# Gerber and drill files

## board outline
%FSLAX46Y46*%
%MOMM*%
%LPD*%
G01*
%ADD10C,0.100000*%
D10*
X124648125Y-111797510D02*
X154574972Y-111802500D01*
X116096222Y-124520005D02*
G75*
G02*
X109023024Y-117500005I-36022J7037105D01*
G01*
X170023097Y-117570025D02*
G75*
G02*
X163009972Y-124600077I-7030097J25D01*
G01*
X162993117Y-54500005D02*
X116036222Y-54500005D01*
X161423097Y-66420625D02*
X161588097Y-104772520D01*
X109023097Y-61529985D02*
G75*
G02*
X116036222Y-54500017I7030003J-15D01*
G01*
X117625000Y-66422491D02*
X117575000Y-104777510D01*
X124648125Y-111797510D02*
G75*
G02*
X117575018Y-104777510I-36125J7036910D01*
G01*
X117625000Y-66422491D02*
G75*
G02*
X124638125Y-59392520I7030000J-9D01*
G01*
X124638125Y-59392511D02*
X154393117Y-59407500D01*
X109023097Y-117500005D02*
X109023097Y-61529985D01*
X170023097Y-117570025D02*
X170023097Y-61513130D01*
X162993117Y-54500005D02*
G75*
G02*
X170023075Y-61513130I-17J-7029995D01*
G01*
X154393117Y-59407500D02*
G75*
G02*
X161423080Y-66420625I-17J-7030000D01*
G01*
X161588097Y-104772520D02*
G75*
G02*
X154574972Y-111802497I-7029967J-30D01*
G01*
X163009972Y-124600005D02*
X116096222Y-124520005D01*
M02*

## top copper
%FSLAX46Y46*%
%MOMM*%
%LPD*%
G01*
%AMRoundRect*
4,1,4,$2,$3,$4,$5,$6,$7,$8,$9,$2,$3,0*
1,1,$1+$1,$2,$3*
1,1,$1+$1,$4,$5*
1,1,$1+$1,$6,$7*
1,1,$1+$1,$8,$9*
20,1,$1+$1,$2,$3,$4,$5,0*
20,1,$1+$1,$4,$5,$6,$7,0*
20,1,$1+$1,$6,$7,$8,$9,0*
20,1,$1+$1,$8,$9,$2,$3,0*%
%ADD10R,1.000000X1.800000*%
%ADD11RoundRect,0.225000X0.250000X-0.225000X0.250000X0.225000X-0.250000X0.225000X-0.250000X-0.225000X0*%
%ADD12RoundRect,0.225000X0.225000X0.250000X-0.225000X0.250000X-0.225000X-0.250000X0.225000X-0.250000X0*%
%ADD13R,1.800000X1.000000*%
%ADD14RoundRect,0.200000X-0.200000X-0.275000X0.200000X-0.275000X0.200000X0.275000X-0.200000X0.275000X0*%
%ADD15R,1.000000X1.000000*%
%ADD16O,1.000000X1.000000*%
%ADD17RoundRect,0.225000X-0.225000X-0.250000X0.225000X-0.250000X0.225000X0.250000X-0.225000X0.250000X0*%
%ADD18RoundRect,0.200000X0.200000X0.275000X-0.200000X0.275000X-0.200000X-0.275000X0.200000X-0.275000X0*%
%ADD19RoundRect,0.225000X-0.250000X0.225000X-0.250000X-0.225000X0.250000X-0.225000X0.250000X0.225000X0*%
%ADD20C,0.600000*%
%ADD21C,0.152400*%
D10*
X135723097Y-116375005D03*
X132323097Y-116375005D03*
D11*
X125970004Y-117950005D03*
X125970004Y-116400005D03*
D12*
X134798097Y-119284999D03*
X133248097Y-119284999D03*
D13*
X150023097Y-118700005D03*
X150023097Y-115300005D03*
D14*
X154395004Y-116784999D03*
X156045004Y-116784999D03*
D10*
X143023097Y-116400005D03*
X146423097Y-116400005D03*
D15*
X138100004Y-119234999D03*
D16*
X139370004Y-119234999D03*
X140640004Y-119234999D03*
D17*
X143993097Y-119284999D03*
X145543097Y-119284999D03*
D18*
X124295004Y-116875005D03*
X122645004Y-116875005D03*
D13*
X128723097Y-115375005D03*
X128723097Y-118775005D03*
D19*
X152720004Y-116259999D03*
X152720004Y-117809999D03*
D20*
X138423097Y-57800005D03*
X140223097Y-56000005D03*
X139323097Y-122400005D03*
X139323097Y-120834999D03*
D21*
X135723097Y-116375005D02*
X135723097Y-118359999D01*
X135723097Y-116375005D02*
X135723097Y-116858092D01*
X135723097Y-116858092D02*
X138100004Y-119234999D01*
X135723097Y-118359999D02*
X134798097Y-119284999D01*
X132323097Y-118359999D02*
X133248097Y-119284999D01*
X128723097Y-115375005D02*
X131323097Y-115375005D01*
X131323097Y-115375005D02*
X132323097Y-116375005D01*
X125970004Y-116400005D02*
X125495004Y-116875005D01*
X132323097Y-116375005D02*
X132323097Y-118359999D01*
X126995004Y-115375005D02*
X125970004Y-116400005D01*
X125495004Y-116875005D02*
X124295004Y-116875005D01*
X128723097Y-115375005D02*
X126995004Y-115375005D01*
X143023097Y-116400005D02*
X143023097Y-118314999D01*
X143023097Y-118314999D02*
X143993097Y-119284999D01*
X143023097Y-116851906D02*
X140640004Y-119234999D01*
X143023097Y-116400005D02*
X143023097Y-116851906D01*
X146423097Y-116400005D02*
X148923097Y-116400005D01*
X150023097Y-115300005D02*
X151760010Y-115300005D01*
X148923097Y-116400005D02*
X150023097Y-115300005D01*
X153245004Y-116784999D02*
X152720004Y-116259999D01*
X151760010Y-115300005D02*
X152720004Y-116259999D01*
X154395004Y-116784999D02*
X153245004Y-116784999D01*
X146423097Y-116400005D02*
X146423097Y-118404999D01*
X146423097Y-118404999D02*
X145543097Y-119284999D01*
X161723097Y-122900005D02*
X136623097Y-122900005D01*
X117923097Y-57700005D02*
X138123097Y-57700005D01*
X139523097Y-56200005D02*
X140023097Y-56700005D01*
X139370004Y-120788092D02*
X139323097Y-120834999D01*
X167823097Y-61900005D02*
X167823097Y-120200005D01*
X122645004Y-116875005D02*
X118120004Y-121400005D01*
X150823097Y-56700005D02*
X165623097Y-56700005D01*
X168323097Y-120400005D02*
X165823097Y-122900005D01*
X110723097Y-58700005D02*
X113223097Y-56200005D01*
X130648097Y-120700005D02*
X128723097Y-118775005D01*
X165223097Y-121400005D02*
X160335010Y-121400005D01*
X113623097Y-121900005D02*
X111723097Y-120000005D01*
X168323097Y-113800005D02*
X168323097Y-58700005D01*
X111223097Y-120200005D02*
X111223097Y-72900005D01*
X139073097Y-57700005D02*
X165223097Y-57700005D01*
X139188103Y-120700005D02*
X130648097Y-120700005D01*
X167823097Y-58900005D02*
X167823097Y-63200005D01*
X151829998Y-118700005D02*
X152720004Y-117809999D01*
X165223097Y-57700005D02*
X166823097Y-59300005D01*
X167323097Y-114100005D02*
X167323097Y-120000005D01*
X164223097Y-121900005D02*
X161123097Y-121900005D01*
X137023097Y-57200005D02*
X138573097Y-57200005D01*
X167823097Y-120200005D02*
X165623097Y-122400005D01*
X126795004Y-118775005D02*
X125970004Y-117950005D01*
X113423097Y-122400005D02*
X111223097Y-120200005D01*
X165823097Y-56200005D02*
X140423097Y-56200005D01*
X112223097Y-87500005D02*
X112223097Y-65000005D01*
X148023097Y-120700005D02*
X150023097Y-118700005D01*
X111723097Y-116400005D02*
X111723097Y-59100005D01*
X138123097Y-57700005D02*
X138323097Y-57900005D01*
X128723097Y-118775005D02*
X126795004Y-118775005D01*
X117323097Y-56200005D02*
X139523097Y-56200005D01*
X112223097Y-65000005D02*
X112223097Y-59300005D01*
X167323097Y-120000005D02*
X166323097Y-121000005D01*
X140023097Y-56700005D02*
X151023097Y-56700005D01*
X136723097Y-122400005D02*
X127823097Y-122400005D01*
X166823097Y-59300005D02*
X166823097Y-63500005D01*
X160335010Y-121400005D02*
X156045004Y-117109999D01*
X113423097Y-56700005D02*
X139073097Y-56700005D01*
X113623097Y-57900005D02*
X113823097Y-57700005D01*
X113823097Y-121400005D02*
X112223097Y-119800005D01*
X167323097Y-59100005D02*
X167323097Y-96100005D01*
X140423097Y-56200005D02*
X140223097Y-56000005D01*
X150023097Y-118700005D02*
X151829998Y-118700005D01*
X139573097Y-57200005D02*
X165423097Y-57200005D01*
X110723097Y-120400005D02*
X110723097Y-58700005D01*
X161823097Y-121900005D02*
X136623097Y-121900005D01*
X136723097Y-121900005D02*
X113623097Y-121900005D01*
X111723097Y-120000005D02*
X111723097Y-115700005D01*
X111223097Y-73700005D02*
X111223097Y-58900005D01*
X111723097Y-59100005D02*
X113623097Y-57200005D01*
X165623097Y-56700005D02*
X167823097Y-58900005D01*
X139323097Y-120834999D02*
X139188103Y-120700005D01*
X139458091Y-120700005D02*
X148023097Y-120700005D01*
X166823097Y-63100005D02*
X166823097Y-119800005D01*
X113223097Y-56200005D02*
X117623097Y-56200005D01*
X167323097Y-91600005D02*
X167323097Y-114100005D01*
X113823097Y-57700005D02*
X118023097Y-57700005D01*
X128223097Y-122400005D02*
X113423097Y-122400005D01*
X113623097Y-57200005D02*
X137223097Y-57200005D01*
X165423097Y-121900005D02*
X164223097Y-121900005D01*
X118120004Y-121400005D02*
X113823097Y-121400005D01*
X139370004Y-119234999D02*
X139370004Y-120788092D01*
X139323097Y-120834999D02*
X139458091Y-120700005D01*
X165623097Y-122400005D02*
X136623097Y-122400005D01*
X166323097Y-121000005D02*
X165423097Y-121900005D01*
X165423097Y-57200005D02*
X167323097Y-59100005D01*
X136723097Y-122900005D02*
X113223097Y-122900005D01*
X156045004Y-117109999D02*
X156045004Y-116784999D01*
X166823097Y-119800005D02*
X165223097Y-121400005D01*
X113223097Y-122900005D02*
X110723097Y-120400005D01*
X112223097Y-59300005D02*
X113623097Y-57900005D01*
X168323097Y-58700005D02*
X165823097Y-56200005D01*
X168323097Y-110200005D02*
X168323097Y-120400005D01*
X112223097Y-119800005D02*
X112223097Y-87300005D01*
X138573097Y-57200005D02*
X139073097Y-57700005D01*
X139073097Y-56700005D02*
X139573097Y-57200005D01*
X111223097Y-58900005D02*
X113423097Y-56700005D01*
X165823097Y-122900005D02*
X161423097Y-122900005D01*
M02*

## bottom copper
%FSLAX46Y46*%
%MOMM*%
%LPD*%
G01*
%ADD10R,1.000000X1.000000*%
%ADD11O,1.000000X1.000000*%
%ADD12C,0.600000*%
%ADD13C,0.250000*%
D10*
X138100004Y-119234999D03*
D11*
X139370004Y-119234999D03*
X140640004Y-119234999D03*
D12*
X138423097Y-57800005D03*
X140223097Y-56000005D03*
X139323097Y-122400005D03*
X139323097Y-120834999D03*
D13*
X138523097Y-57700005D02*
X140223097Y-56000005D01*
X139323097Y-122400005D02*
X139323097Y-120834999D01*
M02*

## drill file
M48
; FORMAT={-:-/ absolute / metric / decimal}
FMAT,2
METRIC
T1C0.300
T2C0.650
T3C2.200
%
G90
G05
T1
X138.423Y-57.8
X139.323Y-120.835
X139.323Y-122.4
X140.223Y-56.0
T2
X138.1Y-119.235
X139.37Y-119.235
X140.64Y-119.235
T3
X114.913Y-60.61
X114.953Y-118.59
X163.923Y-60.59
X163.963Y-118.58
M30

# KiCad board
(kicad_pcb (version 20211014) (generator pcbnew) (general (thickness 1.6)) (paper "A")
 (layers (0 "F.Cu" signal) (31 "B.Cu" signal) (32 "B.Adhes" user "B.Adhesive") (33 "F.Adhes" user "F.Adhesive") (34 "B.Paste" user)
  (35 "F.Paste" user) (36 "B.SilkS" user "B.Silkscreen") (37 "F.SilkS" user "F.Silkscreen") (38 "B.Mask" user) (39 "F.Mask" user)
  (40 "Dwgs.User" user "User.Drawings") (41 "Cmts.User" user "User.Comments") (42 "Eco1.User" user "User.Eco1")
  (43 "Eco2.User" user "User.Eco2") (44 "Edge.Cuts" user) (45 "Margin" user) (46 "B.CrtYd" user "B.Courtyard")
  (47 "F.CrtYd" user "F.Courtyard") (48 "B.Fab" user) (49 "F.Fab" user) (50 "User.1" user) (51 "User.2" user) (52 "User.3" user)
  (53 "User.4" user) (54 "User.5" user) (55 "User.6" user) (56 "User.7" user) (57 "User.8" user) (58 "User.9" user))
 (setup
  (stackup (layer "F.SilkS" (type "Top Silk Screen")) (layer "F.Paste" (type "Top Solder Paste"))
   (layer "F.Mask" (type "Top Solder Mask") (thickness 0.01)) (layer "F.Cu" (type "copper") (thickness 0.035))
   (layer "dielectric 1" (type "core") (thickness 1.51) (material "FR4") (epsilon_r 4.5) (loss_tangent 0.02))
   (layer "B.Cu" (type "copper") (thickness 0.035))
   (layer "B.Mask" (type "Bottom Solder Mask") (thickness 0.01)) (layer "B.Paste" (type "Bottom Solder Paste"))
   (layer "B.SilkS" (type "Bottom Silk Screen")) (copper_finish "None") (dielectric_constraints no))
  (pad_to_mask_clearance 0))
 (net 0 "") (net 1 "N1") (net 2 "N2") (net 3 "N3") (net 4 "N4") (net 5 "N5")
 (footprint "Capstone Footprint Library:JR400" (layer "F.Cu") (at 134.023097 116.375005 180)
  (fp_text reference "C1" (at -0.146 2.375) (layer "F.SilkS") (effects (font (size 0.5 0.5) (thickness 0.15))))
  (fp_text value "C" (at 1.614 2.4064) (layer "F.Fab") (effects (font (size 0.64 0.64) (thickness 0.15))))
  (pad "1" smd rect (at -1.7 0 180) (size 1 1.8) (layers "F.Cu" "F.Paste" "F.Mask") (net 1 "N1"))
  (pad "2" smd rect (at 1.7 0 180) (size 1 1.8) (layers "F.Cu" "F.Paste" "F.Mask") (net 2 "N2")))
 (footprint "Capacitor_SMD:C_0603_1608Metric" (layer "F.Cu") (at 125.970004 117.175005 90)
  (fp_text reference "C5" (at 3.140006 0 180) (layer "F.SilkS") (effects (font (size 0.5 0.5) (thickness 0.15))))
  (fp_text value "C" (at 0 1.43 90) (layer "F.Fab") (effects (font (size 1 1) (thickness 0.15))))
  (pad "1" smd roundrect (at -0.775 0 90) (size 0.9 0.95) (layers "F.Cu" "F.Paste" "F.Mask") (roundrect_rratio 0.25) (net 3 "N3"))
  (pad "2" smd roundrect (at 0.775 0 90) (size 0.9 0.95) (layers "F.Cu" "F.Paste" "F.Mask") (roundrect_rratio 0.25) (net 2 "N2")))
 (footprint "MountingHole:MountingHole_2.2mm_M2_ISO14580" (layer "F.Cu") (at 163.923097 60.590005)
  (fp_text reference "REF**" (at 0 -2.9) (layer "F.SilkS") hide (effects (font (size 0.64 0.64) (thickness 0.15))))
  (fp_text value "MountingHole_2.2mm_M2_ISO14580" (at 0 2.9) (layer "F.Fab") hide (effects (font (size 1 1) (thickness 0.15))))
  (pad "" np_thru_hole circle (at 0 0) (size 2.2 2.2) (drill 2.2) (layers *.Cu *.Mask)))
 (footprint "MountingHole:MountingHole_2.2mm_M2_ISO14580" (layer "F.Cu") (at 163.963097 118.580005)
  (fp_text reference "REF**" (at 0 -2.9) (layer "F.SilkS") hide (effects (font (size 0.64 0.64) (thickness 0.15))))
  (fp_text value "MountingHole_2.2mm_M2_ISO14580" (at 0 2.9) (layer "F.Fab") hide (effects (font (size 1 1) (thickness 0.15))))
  (pad "" np_thru_hole circle (at 0 0) (size 2.2 2.2) (drill 2.2) (layers *.Cu *.Mask)))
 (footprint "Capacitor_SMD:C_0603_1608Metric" (layer "F.Cu") (at 134.023097 119.284999 180)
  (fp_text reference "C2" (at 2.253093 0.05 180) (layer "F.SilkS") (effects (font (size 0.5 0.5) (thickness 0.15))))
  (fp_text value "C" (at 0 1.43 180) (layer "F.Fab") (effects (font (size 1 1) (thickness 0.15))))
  (pad "1" smd roundrect (at -0.775 0 180) (size 0.9 0.95) (layers "F.Cu" "F.Paste" "F.Mask") (roundrect_rratio 0.25) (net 1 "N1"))
  (pad "2" smd roundrect (at 0.775 0 180) (size 0.9 0.95) (layers "F.Cu" "F.Paste" "F.Mask") (roundrect_rratio 0.25) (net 2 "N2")))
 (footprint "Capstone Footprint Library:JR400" (layer "F.Cu") (at 150.023097 117.000005 90)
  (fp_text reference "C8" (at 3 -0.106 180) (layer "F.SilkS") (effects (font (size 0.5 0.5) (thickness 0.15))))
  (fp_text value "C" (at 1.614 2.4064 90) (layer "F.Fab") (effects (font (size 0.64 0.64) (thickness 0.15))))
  (pad "1" smd rect (at -1.7 0 90) (size 1 1.8) (layers "F.Cu" "F.Paste" "F.Mask") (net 3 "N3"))
  (pad "2" smd rect (at 1.7 0 90) (size 1 1.8) (layers "F.Cu" "F.Paste" "F.Mask") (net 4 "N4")))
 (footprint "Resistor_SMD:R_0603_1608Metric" (layer "F.Cu") (at 155.220004 116.784999)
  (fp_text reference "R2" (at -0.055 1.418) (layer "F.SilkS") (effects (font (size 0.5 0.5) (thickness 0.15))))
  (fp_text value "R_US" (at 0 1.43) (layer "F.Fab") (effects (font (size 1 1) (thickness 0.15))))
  (pad "1" smd roundrect (at -0.825 0) (size 0.8 0.95) (layers "F.Cu" "F.Paste" "F.Mask") (roundrect_rratio 0.25) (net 4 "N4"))
  (pad "2" smd roundrect (at 0.825 0) (size 0.8 0.95) (layers "F.Cu" "F.Paste" "F.Mask") (roundrect_rratio 0.25) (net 3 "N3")))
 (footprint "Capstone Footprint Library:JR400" (layer "F.Cu") (at 144.723097 116.400005)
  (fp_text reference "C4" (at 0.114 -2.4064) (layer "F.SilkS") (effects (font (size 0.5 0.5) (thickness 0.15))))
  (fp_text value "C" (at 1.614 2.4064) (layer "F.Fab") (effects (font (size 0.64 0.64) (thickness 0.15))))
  (pad "1" smd rect (at -1.7 0) (size 1 1.8) (layers "F.Cu" "F.Paste" "F.Mask") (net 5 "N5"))
  (pad "2" smd rect (at 1.7 0) (size 1 1.8) (layers "F.Cu" "F.Paste" "F.Mask") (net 4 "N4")))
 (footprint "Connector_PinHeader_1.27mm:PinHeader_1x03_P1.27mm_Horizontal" (layer "F.Cu") (at 138.100004 119.234999 90)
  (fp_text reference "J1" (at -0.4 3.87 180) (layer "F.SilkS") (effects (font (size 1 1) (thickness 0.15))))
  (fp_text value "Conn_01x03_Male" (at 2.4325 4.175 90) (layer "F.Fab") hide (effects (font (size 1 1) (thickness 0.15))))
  (pad "1" thru_hole rect (at 0 0 90) (size 1 1) (drill 0.65) (layers *.Cu *.Mask) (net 1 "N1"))
  (pad "2" thru_hole oval (at 0 1.27 90) (size 1 1) (drill 0.65) (layers *.Cu *.Mask) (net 3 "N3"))
  (pad "3" thru_hole oval (at 0 2.54 90) (size 1 1) (drill 0.65) (layers *.Cu *.Mask) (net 5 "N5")))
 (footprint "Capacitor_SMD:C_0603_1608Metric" (layer "F.Cu") (at 144.768097 119.284999)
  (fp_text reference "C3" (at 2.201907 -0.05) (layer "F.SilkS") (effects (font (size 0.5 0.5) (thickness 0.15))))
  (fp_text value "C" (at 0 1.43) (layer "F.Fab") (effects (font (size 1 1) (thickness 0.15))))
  (pad "1" smd roundrect (at -0.775 0) (size 0.9 0.95) (layers "F.Cu" "F.Paste" "F.Mask") (roundrect_rratio 0.25) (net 5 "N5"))
  (pad "2" smd roundrect (at 0.775 0) (size 0.9 0.95) (layers "F.Cu" "F.Paste" "F.Mask") (roundrect_rratio 0.25) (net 4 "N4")))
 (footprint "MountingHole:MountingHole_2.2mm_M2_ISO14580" (layer "F.Cu") (at 114.953097 118.590005)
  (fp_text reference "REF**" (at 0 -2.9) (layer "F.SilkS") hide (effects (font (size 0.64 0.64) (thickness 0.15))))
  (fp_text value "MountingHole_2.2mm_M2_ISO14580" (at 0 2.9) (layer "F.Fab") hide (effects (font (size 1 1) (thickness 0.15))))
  (pad "" np_thru_hole circle (at 0 0) (size 2.2 2.2) (drill 2.2) (layers *.Cu *.Mask)))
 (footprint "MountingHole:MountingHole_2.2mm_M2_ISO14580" (layer "F.Cu") (at 114.913097 60.610005)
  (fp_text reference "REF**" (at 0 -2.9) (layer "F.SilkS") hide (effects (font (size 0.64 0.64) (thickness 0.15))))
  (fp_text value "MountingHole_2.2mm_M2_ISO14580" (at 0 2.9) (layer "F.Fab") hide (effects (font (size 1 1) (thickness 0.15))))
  (pad "" np_thru_hole circle (at 0 0) (size 2.2 2.2) (drill 2.2) (layers *.Cu *.Mask)))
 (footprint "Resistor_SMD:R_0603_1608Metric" (layer "F.Cu") (at 123.470004 116.875005 180)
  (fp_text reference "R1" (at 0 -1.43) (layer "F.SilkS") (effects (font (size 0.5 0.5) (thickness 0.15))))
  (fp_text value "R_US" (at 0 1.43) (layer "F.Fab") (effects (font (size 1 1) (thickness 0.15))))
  (pad "1" smd roundrect (at -0.825 0 180) (size 0.8 0.95) (layers "F.Cu" "F.Paste" "F.Mask") (roundrect_rratio 0.25) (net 2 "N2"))
  (pad "2" smd roundrect (at 0.825 0 180) (size 0.8 0.95) (layers "F.Cu" "F.Paste" "F.Mask") (roundrect_rratio 0.25) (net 3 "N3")))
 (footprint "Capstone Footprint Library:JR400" (layer "F.Cu") (at 128.723097 117.075005 -90)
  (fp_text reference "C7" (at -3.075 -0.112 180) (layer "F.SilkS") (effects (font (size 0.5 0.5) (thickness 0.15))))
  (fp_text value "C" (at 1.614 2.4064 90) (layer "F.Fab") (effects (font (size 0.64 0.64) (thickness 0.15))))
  (pad "1" smd rect (at -1.7 0 270) (size 1 1.8) (layers "F.Cu" "F.Paste" "F.Mask") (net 2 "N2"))
  (pad "2" smd rect (at 1.7 0 270) (size 1 1.8) (layers "F.Cu" "F.Paste" "F.Mask") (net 3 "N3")))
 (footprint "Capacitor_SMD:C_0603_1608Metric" (layer "F.Cu") (at 152.720004 117.034999 -90)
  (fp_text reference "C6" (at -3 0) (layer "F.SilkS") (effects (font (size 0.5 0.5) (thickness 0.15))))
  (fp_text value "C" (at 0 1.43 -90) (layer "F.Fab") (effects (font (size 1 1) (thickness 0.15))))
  (pad "1" smd roundrect (at -0.775 0 270) (size 0.9 0.95) (layers "F.Cu" "F.Paste" "F.Mask") (roundrect_rratio 0.25) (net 4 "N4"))
  (pad "2" smd roundrect (at 0.775 0 270) (size 0.9 0.95) (layers "F.Cu" "F.Paste" "F.Mask") (roundrect_rratio 0.25) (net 3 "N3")))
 (gr_line (start 124.648125 111.79751) (end 154.574972 111.8025) (layer "Edge.Cuts") (width 0.1))
 (gr_arc (start 116.096222 124.520005) (mid 111.103006 122.47769) (end 109.023097 117.500005) (layer "Edge.Cuts") (width 0.1))
 (gr_arc (start 170.023097 117.570025) (mid 167.970004 122.535002) (end 163.009972 124.600005) (layer "Edge.Cuts") (width 0.1))
 (gr_line (start 162.993117 54.500005) (end 116.036222 54.500005) (layer "Edge.Cuts") (width 0.1))
 (gr_line (start 161.423097 66.420625) (end 161.588097 104.77252) (layer "Edge.Cuts") (width 0.1))
 (gr_arc (start 109.023097 61.529985) (mid 111.076178 56.565001) (end 116.036222 54.500005) (layer "Edge.Cuts") (width 0.1))
 (gr_line (start 117.625 66.422491) (end 117.575 104.77751) (layer "Edge.Cuts") (width 0.1))
 (gr_arc (start 124.648125 111.79751) (mid 119.654876 109.755226) (end 117.575 104.77751) (layer "Edge.Cuts") (width 0.1))
 (gr_arc (start 117.625 66.422491) (mid 119.678079 61.457504) (end 124.638125 59.392511) (layer "Edge.Cuts") (width 0.1))
 (gr_line (start 124.638125 59.392511) (end 154.393117 59.4075) (layer "Edge.Cuts") (width 0.1))
 (gr_line (start 109.023097 117.500005) (end 109.023097 61.529985) (layer "Edge.Cuts") (width 0.1))
 (gr_line (start 170.023097 117.570025) (end 170.023097 61.51313) (layer "Edge.Cuts") (width 0.1))
 (gr_arc (start 162.993117 54.500005) (mid 167.958097 56.553087) (end 170.023097 61.51313) (layer "Edge.Cuts") (width 0.1))
 (gr_arc (start 154.393117 59.4075) (mid 159.358099 61.460581) (end 161.423097 66.420625) (layer "Edge.Cuts") (width 0.1))
 (gr_arc (start 161.588097 104.77252) (mid 159.535019 109.73753) (end 154.574972 111.8025) (layer "Edge.Cuts") (width 0.1))
 (gr_line (start 163.009972 124.600005) (end 116.096222 124.520005) (layer "Edge.Cuts") (width 0.1))
 (segment (start 135.723097 116.375005) (end 135.723097 118.359999) (width 0.1524) (layer "F.Cu") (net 1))
 (segment (start 135.723097 116.375005) (end 135.723097 116.858092) (width 0.1524) (layer "F.Cu") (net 1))
 (segment (start 135.723097 116.858092) (end 138.100004 119.234999) (width 0.1524) (layer "F.Cu") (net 1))
 (segment (start 135.723097 118.359999) (end 134.798097 119.284999) (width 0.1524) (layer "F.Cu") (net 1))
 (segment (start 132.323097 118.359999) (end 133.248097 119.284999) (width 0.1524) (layer "F.Cu") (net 2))
 (segment (start 128.723097 115.375005) (end 131.323097 115.375005) (width 0.1524) (layer "F.Cu") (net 2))
 (segment (start 131.323097 115.375005) (end 132.323097 116.375005) (width 0.1524) (layer "F.Cu") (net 2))
 (segment (start 125.970004 116.400005) (end 125.495004 116.875005) (width 0.1524) (layer "F.Cu") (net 2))
 (segment (start 132.323097 116.375005) (end 132.323097 118.359999) (width 0.1524) (layer "F.Cu") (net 2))
 (segment (start 126.995004 115.375005) (end 125.970004 116.400005) (width 0.1524) (layer "F.Cu") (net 2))
 (segment (start 125.495004 116.875005) (end 124.295004 116.875005) (width 0.1524) (layer "F.Cu") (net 2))
 (segment (start 128.723097 115.375005) (end 126.995004 115.375005) (width 0.1524) (layer "F.Cu") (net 2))
 (segment (start 143.023097 116.400005) (end 143.023097 118.314999) (width 0.1524) (layer "F.Cu") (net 5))
 (segment (start 143.023097 118.314999) (end 143.993097 119.284999) (width 0.1524) (layer "F.Cu") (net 5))
 (segment (start 143.023097 116.851906) (end 140.640004 119.234999) (width 0.1524) (layer "F.Cu") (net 5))
 (segment (start 143.023097 116.400005) (end 143.023097 116.851906) (width 0.1524) (layer "F.Cu") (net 5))
 (segment (start 146.423097 116.400005) (end 148.923097 116.400005) (width 0.1524) (layer "F.Cu") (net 4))
 (segment (start 150.023097 115.300005) (end 151.76001 115.300005) (width 0.1524) (layer "F.Cu") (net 4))
 (segment (start 148.923097 116.400005) (end 150.023097 115.300005) (width 0.1524) (layer "F.Cu") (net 4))
 (segment (start 153.245004 116.784999) (end 152.720004 116.259999) (width 0.1524) (layer "F.Cu") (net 4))
 (segment (start 151.76001 115.300005) (end 152.720004 116.259999) (width 0.1524) (layer "F.Cu") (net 4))
 (segment (start 154.395004 116.784999) (end 153.245004 116.784999) (width 0.1524) (layer "F.Cu") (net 4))
 (segment (start 146.423097 116.400005) (end 146.423097 118.404999) (width 0.1524) (layer "F.Cu") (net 4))
 (segment (start 146.423097 118.404999) (end 145.543097 119.284999) (width 0.1524) (layer "F.Cu") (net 4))
 (segment (start 161.723097 122.900005) (end 136.623097 122.900005) (width 0.1524) (layer "F.Cu") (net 3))
 (segment (start 117.923097 57.700005) (end 138.123097 57.700005) (width 0.1524) (layer "F.Cu") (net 3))
 (segment (start 139.523097 56.200005) (end 140.023097 56.700005) (width 0.1524) (layer "F.Cu") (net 3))
 (segment (start 139.370004 120.788092) (end 139.323097 120.834999) (width 0.1524) (layer "F.Cu") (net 3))
 (segment (start 167.823097 61.900005) (end 167.823097 120.200005) (width 0.1524) (layer "F.Cu") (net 3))
 (segment (start 122.645004 116.875005) (end 118.120004 121.400005) (width 0.1524) (layer "F.Cu") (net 3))
 (segment (start 150.823097 56.700005) (end 165.623097 56.700005) (width 0.1524) (layer "F.Cu") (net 3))
 (segment (start 168.323097 120.400005) (end 165.823097 122.900005) (width 0.1524) (layer "F.Cu") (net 3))
 (segment (start 110.723097 58.700005) (end 113.223097 56.200005) (width 0.1524) (layer "F.Cu") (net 3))
 (segment (start 130.648097 120.700005) (end 128.723097 118.775005) (width 0.1524) (layer "F.Cu") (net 3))
 (segment (start 165.223097 121.400005) (end 160.33501 121.400005) (width 0.1524) (layer "F.Cu") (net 3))
 (segment (start 113.623097 121.900005) (end 111.723097 120.000005) (width 0.1524) (layer "F.Cu") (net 3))
 (segment (start 168.323097 113.800005) (end 168.323097 58.700005) (width 0.1524) (layer "F.Cu") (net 3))
 (segment (start 111.223097 120.200005) (end 111.223097 72.900005) (width 0.1524) (layer "F.Cu") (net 3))
 (segment (start 139.073097 57.700005) (end 165.223097 57.700005) (width 0.1524) (layer "F.Cu") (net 3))
 (segment (start 139.188103 120.700005) (end 130.648097 120.700005) (width 0.1524) (layer "F.Cu") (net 3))
 (segment (start 167.823097 58.900005) (end 167.823097 63.200005) (width 0.1524) (layer "F.Cu") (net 3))
 (segment (start 151.829998 118.700005) (end 152.720004 117.809999) (width 0.1524) (layer "F.Cu") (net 3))
 (segment (start 165.223097 57.700005) (end 166.823097 59.300005) (width 0.1524) (layer "F.Cu") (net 3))
 (segment (start 167.323097 114.100005) (end 167.323097 120.000005) (width 0.1524) (layer "F.Cu") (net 3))
 (segment (start 164.223097 121.900005) (end 161.123097 121.900005) (width 0.1524) (layer "F.Cu") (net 3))
 (segment (start 137.023097 57.200005) (end 138.573097 57.200005) (width 0.1524) (layer "F.Cu") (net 3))
 (segment (start 167.823097 120.200005) (end 165.623097 122.400005) (width 0.1524) (layer "F.Cu") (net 3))
 (segment (start 126.795004 118.775005) (end 125.970004 117.950005) (width 0.1524) (layer "F.Cu") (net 3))
 (segment (start 113.423097 122.400005) (end 111.223097 120.200005) (width 0.1524) (layer "F.Cu") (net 3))
 (segment (start 165.823097 56.200005) (end 140.423097 56.200005) (width 0.1524) (layer "F.Cu") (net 3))
 (segment (start 112.223097 87.500005) (end 112.223097 65.000005) (width 0.1524) (layer "F.Cu") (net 3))
 (segment (start 148.023097 120.700005) (end 150.023097 118.700005) (width 0.1524) (layer "F.Cu") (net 3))
 (segment (start 111.723097 116.400005) (end 111.723097 59.100005) (width 0.1524) (layer "F.Cu") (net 3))
 (segment (start 138.123097 57.700005) (end 138.323097 57.900005) (width 0.1524) (layer "F.Cu") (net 3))
 (segment (start 128.723097 118.775005) (end 126.795004 118.775005) (width 0.1524) (layer "F.Cu") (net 3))
 (segment (start 117.323097 56.200005) (end 139.523097 56.200005) (width 0.1524) (layer "F.Cu") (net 3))
 (segment (start 112.223097 65.000005) (end 112.223097 59.300005) (width 0.1524) (layer "F.Cu") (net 3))
 (segment (start 167.323097 120.000005) (end 166.323097 121.000005) (width 0.1524) (layer "F.Cu") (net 3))
 (segment (start 140.023097 56.700005) (end 151.023097 56.700005) (width 0.1524) (layer "F.Cu") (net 3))
 (segment (start 136.723097 122.400005) (end 127.823097 122.400005) (width 0.1524) (layer "F.Cu") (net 3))
 (segment (start 166.823097 59.300005) (end 166.823097 63.500005) (width 0.1524) (layer "F.Cu") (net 3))
 (segment (start 160.33501 121.400005) (end 156.045004 117.109999) (width 0.1524) (layer "F.Cu") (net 3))
 (segment (start 113.423097 56.700005) (end 139.073097 56.700005) (width 0.1524) (layer "F.Cu") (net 3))
 (segment (start 113.623097 57.900005) (end 113.823097 57.700005) (width 0.1524) (layer "F.Cu") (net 3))
 (segment (start 113.823097 121.400005) (end 112.223097 119.800005) (width 0.1524) (layer "F.Cu") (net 3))
 (segment (start 167.323097 59.100005) (end 167.323097 96.100005) (width 0.1524) (layer "F.Cu") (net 3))
 (segment (start 140.423097 56.200005) (end 140.223097 56.000005) (width 0.1524) (layer "F.Cu") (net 3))
 (segment (start 150.023097 118.700005) (end 151.829998 118.700005) (width 0.1524) (layer "F.Cu") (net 3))
 (segment (start 139.573097 57.200005) (end 165.423097 57.200005) (width 0.1524) (layer "F.Cu") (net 3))
 (segment (start 110.723097 120.400005) (end 110.723097 58.700005) (width 0.1524) (layer "F.Cu") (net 3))
 (segment (start 161.823097 121.900005) (end 136.623097 121.900005) (width 0.1524) (layer "F.Cu") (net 3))
 (segment (start 136.723097 121.900005) (end 113.623097 121.900005) (width 0.1524) (layer "F.Cu") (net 3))
 (segment (start 111.723097 120.000005) (end 111.723097 115.700005) (width 0.1524) (layer "F.Cu") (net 3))
 (segment (start 111.223097 73.700005) (end 111.223097 58.900005) (width 0.1524) (layer "F.Cu") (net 3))
 (segment (start 111.723097 59.100005) (end 113.623097 57.200005) (width 0.1524) (layer "F.Cu") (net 3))
 (segment (start 165.623097 56.700005) (end 167.823097 58.900005) (width 0.1524) (layer "F.Cu") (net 3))
 (segment (start 139.323097 120.834999) (end 139.188103 120.700005) (width 0.1524) (layer "F.Cu") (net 3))
 (segment (start 139.458091 120.700005) (end 148.023097 120.700005) (width 0.1524) (layer "F.Cu") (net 3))
 (segment (start 166.823097 63.100005) (end 166.823097 119.800005) (width 0.1524) (layer "F.Cu") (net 3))
 (segment (start 113.223097 56.200005) (end 117.623097 56.200005) (width 0.1524) (layer "F.Cu") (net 3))
 (segment (start 167.323097 91.600005) (end 167.323097 114.100005) (width 0.1524) (layer "F.Cu") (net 3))
 (segment (start 113.823097 57.700005) (end 118.023097 57.700005) (width 0.1524) (layer "F.Cu") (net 3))
 (segment (start 128.223097 122.400005) (end 113.423097 122.400005) (width 0.1524) (layer "F.Cu") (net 3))
 (segment (start 113.623097 57.200005) (end 137.223097 57.200005) (width 0.1524) (layer "F.Cu") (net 3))
 (segment (start 165.423097 121.900005) (end 164.223097 121.900005) (width 0.1524) (layer "F.Cu") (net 3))
 (segment (start 118.120004 121.400005) (end 113.823097 121.400005) (width 0.1524) (layer "F.Cu") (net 3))
 (segment (start 139.370004 119.234999) (end 139.370004 120.788092) (width 0.1524) (layer "F.Cu") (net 3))
 (segment (start 139.323097 120.834999) (end 139.458091 120.700005) (width 0.1524) (layer "F.Cu") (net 3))
 (segment (start 165.623097 122.400005) (end 136.623097 122.400005) (width 0.1524) (layer "F.Cu") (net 3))
 (segment (start 166.323097 121.000005) (end 165.423097 121.900005) (width 0.1524) (layer "F.Cu") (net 3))
 (segment (start 165.423097 57.200005) (end 167.323097 59.100005) (width 0.1524) (layer "F.Cu") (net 3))
 (segment (start 136.723097 122.900005) (end 113.223097 122.900005) (width 0.1524) (layer "F.Cu") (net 3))
 (segment (start 156.045004 117.109999) (end 156.045004 116.784999) (width 0.1524) (layer "F.Cu") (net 3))
 (segment (start 166.823097 119.800005) (end 165.223097 121.400005) (width 0.1524) (layer "F.Cu") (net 3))
 (segment (start 113.223097 122.900005) (end 110.723097 120.400005) (width 0.1524) (layer "F.Cu") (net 3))
 (segment (start 112.223097 59.300005) (end 113.623097 57.900005) (width 0.1524) (layer "F.Cu") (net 3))
 (segment (start 168.323097 58.700005) (end 165.823097 56.200005) (width 0.1524) (layer "F.Cu") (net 3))
 (segment (start 168.323097 110.200005) (end 168.323097 120.400005) (width 0.1524) (layer "F.Cu") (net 3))
 (segment (start 112.223097 119.800005) (end 112.223097 87.300005) (width 0.1524) (layer "F.Cu") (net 3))
 (segment (start 138.573097 57.200005) (end 139.073097 57.700005) (width 0.1524) (layer "F.Cu") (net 3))
 (segment (start 139.073097 56.700005) (end 139.573097 57.200005) (width 0.1524) (layer "F.Cu") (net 3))
 (segment (start 111.223097 58.900005) (end 113.423097 56.700005) (width 0.1524) (layer "F.Cu") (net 3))
 (segment (start 165.823097 122.900005) (end 161.423097 122.900005) (width 0.1524) (layer "F.Cu") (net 3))
 (via (at 138.423097 57.800005) (size 0.6) (drill 0.3) (layers "F.Cu" "B.Cu") (free) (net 3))
 (via (at 140.223097 56.000005) (size 0.6) (drill 0.3) (layers "F.Cu" "B.Cu") (free) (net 3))
 (via (at 139.323097 122.400005) (size 0.6) (drill 0.3) (layers "F.Cu" "B.Cu") (free) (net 3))
 (via (at 139.323097 120.834999) (size 0.6) (drill 0.3) (layers "F.Cu" "B.Cu") (free) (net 3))
 (segment (start 138.523097 57.700005) (end 140.223097 56.000005) (width 0.25) (layer "B.Cu") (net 3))
 (segment (start 139.323097 122.400005) (end 139.323097 120.834999) (width 0.25) (layer "B.Cu") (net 3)))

